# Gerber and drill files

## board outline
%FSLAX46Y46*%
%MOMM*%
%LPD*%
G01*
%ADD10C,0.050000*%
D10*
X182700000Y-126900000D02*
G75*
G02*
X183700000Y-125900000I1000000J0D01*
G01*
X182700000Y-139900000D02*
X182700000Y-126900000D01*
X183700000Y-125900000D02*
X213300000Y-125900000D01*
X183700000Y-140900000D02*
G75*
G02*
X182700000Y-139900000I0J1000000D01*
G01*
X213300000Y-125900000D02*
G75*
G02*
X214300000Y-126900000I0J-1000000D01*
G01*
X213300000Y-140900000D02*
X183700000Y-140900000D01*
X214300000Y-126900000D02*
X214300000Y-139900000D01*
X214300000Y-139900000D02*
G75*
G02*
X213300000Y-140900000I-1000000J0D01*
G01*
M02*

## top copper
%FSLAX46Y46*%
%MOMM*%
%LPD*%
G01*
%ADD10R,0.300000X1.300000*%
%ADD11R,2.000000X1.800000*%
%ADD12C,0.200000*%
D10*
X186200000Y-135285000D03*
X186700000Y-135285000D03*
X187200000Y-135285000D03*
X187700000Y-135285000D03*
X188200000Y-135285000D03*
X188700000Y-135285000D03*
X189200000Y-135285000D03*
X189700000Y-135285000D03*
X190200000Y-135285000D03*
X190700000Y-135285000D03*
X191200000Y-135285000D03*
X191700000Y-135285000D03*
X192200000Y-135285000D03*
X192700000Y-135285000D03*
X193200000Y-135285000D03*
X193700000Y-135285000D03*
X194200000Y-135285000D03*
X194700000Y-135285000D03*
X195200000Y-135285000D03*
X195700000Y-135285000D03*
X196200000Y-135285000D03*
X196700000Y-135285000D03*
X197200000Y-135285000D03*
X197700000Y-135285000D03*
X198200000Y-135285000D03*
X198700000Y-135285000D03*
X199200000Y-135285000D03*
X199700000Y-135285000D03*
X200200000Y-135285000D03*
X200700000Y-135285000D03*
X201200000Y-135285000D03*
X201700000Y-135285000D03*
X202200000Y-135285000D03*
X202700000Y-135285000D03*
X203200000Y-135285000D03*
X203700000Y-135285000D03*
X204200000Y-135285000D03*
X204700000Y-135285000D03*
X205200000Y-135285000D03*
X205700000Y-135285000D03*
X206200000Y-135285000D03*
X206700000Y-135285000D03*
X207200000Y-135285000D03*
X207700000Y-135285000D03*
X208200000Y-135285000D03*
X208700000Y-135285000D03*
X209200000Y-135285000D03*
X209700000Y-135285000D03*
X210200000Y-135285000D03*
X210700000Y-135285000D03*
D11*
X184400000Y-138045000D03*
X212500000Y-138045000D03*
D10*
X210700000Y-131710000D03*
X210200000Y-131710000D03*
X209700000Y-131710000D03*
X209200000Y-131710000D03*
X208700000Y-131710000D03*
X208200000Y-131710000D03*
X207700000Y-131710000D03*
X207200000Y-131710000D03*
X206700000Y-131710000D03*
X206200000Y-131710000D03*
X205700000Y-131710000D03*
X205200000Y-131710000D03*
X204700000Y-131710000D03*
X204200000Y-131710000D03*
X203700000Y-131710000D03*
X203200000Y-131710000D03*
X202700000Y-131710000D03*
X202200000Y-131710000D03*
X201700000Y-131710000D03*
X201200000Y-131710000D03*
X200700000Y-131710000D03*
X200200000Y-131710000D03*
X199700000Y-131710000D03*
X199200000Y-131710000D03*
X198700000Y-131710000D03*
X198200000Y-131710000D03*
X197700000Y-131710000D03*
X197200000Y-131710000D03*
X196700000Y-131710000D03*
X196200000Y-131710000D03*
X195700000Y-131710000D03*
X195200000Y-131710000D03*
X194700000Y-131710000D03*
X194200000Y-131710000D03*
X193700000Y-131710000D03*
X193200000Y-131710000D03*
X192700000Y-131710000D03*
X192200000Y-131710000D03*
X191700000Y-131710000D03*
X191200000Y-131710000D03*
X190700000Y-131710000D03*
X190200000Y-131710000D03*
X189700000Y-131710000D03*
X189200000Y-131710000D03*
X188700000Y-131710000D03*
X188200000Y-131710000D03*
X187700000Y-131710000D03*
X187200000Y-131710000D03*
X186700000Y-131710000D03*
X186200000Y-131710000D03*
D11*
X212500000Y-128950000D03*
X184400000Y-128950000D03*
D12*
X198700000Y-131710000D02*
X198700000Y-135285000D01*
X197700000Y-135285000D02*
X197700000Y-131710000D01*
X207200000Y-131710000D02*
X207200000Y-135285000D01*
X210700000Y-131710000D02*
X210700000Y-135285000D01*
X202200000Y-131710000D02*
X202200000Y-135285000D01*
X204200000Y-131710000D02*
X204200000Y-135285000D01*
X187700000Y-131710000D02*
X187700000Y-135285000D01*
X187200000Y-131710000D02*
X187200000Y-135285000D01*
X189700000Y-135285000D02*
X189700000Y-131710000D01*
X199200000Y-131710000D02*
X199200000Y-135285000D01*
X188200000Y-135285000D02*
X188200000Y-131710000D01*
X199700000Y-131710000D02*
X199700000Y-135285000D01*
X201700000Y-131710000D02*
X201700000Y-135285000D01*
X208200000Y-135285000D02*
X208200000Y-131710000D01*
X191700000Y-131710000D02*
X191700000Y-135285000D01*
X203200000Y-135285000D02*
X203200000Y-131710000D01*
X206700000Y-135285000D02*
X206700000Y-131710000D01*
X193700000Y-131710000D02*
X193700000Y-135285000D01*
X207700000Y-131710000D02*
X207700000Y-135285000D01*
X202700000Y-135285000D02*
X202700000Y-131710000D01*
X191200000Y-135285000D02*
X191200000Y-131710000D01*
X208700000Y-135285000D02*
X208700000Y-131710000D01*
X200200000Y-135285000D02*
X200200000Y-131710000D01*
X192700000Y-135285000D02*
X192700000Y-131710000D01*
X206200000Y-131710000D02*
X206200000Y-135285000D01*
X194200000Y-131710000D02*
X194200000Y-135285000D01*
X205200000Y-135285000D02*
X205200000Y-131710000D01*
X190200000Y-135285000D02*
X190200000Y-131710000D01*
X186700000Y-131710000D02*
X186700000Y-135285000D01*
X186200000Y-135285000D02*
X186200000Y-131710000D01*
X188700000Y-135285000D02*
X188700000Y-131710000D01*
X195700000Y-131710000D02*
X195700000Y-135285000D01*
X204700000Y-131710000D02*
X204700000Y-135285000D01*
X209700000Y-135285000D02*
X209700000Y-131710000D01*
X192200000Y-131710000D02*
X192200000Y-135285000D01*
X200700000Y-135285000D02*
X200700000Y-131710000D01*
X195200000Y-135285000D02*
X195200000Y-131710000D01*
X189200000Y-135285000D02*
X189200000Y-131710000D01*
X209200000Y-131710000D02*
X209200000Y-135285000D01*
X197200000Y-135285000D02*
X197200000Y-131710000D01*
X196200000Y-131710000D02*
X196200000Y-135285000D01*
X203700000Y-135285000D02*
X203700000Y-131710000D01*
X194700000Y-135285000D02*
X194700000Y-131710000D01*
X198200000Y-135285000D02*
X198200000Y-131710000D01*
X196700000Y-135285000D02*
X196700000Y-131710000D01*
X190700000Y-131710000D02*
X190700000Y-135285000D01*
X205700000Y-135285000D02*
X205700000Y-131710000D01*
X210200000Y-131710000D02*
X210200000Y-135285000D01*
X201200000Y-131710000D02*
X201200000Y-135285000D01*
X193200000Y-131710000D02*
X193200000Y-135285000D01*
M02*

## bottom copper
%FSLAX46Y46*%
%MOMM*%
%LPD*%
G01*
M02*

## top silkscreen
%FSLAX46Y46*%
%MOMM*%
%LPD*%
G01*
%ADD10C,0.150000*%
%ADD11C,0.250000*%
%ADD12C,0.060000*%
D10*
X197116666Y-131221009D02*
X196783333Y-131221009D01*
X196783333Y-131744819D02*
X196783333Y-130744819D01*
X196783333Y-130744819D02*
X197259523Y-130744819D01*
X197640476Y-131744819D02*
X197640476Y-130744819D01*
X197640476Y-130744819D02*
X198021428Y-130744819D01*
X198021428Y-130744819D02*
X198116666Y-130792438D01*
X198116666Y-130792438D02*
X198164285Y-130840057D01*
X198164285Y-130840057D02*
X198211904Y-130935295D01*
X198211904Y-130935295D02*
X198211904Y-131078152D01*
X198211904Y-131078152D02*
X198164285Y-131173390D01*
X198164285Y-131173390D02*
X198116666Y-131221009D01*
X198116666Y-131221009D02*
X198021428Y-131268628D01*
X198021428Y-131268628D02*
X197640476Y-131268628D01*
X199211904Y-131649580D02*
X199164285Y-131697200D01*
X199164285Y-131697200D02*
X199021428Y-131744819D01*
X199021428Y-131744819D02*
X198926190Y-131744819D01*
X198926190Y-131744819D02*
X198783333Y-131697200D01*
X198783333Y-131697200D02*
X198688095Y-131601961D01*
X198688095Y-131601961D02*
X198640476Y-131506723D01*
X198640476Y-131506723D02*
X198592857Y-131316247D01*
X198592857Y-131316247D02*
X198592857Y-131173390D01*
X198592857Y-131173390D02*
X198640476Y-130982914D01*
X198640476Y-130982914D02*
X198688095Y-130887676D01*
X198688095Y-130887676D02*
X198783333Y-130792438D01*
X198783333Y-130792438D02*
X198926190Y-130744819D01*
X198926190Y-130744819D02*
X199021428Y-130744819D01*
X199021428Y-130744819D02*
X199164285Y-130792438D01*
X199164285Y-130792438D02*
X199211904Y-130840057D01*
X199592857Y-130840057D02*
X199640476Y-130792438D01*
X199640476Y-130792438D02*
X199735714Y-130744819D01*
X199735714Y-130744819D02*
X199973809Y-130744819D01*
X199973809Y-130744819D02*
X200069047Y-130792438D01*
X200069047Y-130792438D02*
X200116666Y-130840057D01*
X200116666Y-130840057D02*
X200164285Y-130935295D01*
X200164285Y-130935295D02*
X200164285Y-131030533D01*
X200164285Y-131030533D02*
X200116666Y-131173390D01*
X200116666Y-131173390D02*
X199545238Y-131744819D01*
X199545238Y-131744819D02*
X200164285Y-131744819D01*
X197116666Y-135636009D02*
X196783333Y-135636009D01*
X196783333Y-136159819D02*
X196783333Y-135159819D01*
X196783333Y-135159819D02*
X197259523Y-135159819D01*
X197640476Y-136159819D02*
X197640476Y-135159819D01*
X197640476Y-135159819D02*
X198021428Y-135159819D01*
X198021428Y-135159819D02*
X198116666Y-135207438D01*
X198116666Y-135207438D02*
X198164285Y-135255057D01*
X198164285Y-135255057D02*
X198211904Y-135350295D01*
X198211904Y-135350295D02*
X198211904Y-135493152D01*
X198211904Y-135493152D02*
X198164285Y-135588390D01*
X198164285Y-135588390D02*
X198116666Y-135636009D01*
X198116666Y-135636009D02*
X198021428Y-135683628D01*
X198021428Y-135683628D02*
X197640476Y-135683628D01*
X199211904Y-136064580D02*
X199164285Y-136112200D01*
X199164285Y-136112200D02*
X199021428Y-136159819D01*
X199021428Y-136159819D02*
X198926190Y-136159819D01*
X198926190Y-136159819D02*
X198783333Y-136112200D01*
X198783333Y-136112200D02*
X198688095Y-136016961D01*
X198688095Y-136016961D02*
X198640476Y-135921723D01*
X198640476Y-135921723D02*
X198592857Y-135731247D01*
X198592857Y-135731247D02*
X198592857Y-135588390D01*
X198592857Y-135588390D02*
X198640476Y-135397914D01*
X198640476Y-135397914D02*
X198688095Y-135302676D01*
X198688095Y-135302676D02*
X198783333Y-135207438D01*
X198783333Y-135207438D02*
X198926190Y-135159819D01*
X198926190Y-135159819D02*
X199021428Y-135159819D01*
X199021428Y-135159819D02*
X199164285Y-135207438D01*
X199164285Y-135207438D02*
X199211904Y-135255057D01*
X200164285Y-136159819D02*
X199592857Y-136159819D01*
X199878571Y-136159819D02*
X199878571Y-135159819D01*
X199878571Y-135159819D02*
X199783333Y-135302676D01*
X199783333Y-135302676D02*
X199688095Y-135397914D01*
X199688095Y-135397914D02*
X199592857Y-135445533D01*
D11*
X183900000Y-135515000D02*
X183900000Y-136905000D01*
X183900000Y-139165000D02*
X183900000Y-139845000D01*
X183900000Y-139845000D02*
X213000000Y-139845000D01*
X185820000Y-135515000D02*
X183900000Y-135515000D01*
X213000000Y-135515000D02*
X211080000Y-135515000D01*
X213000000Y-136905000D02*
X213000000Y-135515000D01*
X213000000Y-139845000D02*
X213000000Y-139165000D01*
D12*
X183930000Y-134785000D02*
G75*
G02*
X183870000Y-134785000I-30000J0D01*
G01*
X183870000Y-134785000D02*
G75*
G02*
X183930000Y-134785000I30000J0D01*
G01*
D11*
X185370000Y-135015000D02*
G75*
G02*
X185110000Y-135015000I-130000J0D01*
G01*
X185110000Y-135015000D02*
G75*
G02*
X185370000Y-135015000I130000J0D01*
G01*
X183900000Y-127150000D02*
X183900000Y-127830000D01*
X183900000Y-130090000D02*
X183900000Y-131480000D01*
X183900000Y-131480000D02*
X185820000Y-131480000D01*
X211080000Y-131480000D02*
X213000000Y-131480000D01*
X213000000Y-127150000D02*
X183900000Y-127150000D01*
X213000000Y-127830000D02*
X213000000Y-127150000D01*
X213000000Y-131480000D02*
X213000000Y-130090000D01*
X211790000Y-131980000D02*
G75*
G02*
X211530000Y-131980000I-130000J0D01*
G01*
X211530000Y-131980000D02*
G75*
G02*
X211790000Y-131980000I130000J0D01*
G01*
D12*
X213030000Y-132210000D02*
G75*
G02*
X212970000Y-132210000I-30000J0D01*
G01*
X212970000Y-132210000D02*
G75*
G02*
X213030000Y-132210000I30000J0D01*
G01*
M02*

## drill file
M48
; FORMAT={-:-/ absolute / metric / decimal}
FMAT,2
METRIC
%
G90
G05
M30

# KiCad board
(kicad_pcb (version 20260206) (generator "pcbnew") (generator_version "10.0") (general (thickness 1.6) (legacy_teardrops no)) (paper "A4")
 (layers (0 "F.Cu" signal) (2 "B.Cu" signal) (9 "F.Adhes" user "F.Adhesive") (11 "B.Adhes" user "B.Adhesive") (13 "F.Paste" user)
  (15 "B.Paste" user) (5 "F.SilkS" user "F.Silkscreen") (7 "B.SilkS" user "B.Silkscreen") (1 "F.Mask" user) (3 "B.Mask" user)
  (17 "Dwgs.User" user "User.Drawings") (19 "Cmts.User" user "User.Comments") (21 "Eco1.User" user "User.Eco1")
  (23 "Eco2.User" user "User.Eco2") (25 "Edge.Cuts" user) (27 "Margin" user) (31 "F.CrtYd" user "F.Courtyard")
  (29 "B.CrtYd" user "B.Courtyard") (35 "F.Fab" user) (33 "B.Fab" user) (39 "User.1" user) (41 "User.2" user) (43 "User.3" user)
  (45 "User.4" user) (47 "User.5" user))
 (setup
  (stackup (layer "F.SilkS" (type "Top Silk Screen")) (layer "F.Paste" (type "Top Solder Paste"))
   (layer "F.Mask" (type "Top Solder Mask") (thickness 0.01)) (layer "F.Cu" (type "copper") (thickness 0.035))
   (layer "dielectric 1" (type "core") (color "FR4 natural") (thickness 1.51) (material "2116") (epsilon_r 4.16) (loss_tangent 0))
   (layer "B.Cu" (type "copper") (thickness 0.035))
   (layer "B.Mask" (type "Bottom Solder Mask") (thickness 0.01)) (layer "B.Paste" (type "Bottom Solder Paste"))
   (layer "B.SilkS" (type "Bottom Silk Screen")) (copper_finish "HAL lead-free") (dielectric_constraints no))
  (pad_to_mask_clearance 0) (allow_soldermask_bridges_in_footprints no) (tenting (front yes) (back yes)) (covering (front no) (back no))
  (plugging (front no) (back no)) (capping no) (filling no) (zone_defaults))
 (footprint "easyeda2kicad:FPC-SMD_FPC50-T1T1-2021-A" (layer "F.Cu") (at 198.45 136.665)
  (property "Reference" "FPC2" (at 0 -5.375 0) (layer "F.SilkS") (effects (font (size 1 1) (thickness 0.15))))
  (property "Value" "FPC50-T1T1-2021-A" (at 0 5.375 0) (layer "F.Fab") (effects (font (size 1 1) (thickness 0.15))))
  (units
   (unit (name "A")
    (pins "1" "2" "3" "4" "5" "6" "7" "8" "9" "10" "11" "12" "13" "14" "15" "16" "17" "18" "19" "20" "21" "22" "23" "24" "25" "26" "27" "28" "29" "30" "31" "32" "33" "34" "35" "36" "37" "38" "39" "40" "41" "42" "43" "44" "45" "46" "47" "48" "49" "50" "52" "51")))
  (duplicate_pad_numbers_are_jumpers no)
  (fp_line (start -14.55 -1.15) (end -14.55 0.24) (stroke (width 0.25) (type solid)) (layer "F.SilkS"))
  (fp_line (start -14.55 2.5) (end -14.55 3.18) (stroke (width 0.25) (type solid)) (layer "F.SilkS"))
  (fp_line (start -14.55 3.18) (end 14.55 3.18) (stroke (width 0.25) (type solid)) (layer "F.SilkS"))
  (fp_line (start -12.63 -1.15) (end -14.55 -1.15) (stroke (width 0.25) (type solid)) (layer "F.SilkS"))
  (fp_line (start 14.55 -1.15) (end 12.63 -1.15) (stroke (width 0.25) (type solid)) (layer "F.SilkS"))
  (fp_line (start 14.55 0.24) (end 14.55 -1.15) (stroke (width 0.25) (type solid)) (layer "F.SilkS"))
  (fp_line (start 14.55 3.18) (end 14.55 2.5) (stroke (width 0.25) (type solid)) (layer "F.SilkS"))
  (fp_circle (center -14.55 -1.88) (end -14.52 -1.88) (stroke (width 0.06) (type solid)) (fill no) (layer "F.SilkS"))
  (fp_circle (center -13.21 -1.65) (end -13.08 -1.65) (stroke (width 0.25) (type solid)) (fill no) (layer "F.SilkS"))
  (pad "1" smd rect (at -12.25 -1.38 180) (size 0.3 1.3) (layers "F.Cu" "F.Mask" "F.Paste") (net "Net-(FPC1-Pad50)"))
  (pad "2" smd rect (at -11.75 -1.38 180) (size 0.3 1.3) (layers "F.Cu" "F.Mask" "F.Paste") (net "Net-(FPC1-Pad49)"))
  (pad "3" smd rect (at -11.25 -1.38 180) (size 0.3 1.3) (layers "F.Cu" "F.Mask" "F.Paste") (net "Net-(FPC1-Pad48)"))
  (pad "4" smd rect (at -10.75 -1.38 180) (size 0.3 1.3) (layers "F.Cu" "F.Mask" "F.Paste") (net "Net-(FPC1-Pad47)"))
  (pad "5" smd rect (at -10.25 -1.38 180) (size 0.3 1.3) (layers "F.Cu" "F.Mask" "F.Paste") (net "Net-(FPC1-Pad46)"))
  (pad "6" smd rect (at -9.75 -1.38 180) (size 0.3 1.3) (layers "F.Cu" "F.Mask" "F.Paste") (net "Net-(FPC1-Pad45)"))
  (pad "7" smd rect (at -9.25 -1.38 180) (size 0.3 1.3) (layers "F.Cu" "F.Mask" "F.Paste") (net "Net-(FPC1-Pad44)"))
  (pad "8" smd rect (at -8.75 -1.38 180) (size 0.3 1.3) (layers "F.Cu" "F.Mask" "F.Paste") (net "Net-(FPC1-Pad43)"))
  (pad "9" smd rect (at -8.25 -1.38 180) (size 0.3 1.3) (layers "F.Cu" "F.Mask" "F.Paste") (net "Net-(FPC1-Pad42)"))
  (pad "10" smd rect (at -7.75 -1.38 180) (size 0.3 1.3) (layers "F.Cu" "F.Mask" "F.Paste") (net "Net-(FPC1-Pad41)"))
  (pad "11" smd rect (at -7.25 -1.38 180) (size 0.3 1.3) (layers "F.Cu" "F.Mask" "F.Paste") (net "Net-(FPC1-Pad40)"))
  (pad "12" smd rect (at -6.75 -1.38 180) (size 0.3 1.3) (layers "F.Cu" "F.Mask" "F.Paste") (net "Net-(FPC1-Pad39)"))
  (pad "13" smd rect (at -6.25 -1.38 180) (size 0.3 1.3) (layers "F.Cu" "F.Mask" "F.Paste") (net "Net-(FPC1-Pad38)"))
  (pad "14" smd rect (at -5.75 -1.38 180) (size 0.3 1.3) (layers "F.Cu" "F.Mask" "F.Paste") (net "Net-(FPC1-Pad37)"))
  (pad "15" smd rect (at -5.25 -1.38 180) (size 0.3 1.3) (layers "F.Cu" "F.Mask" "F.Paste") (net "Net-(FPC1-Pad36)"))
  (pad "16" smd rect (at -4.75 -1.38 180) (size 0.3 1.3) (layers "F.Cu" "F.Mask" "F.Paste") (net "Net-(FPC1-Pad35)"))
  (pad "17" smd rect (at -4.25 -1.38 180) (size 0.3 1.3) (layers "F.Cu" "F.Mask" "F.Paste") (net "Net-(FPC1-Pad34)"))
  (pad "18" smd rect (at -3.75 -1.38 180) (size 0.3 1.3) (layers "F.Cu" "F.Mask" "F.Paste") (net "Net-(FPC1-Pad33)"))
  (pad "19" smd rect (at -3.25 -1.38 180) (size 0.3 1.3) (layers "F.Cu" "F.Mask" "F.Paste") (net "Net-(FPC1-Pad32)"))
  (pad "20" smd rect (at -2.75 -1.38 180) (size 0.3 1.3) (layers "F.Cu" "F.Mask" "F.Paste") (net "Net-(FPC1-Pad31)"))
  (pad "21" smd rect (at -2.25 -1.38 180) (size 0.3 1.3) (layers "F.Cu" "F.Mask" "F.Paste") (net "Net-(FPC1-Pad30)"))
  (pad "22" smd rect (at -1.75 -1.38 180) (size 0.3 1.3) (layers "F.Cu" "F.Mask" "F.Paste") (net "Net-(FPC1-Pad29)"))
  (pad "23" smd rect (at -1.25 -1.38 180) (size 0.3 1.3) (layers "F.Cu" "F.Mask" "F.Paste") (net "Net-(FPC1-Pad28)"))
  (pad "24" smd rect (at -0.75 -1.38 180) (size 0.3 1.3) (layers "F.Cu" "F.Mask" "F.Paste") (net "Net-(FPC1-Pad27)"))
  (pad "25" smd rect (at -0.25 -1.38 180) (size 0.3 1.3) (layers "F.Cu" "F.Mask" "F.Paste") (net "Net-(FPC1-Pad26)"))
  (pad "26" smd rect (at 0.25 -1.38 180) (size 0.3 1.3) (layers "F.Cu" "F.Mask" "F.Paste") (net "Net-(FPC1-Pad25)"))
  (pad "27" smd rect (at 0.75 -1.38 180) (size 0.3 1.3) (layers "F.Cu" "F.Mask" "F.Paste") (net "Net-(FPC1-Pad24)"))
  (pad "28" smd rect (at 1.25 -1.38 180) (size 0.3 1.3) (layers "F.Cu" "F.Mask" "F.Paste") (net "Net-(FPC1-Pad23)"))
  (pad "29" smd rect (at 1.75 -1.38 180) (size 0.3 1.3) (layers "F.Cu" "F.Mask" "F.Paste") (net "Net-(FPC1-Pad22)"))
  (pad "30" smd rect (at 2.25 -1.38 180) (size 0.3 1.3) (layers "F.Cu" "F.Mask" "F.Paste") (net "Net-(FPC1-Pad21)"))
  (pad "31" smd rect (at 2.75 -1.38 180) (size 0.3 1.3) (layers "F.Cu" "F.Mask" "F.Paste") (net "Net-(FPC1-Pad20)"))
  (pad "32" smd rect (at 3.25 -1.38 180) (size 0.3 1.3) (layers "F.Cu" "F.Mask" "F.Paste") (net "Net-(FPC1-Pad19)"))
  (pad "33" smd rect (at 3.75 -1.38 180) (size 0.3 1.3) (layers "F.Cu" "F.Mask" "F.Paste") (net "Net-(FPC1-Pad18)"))
  (pad "34" smd rect (at 4.25 -1.38 180) (size 0.3 1.3) (layers "F.Cu" "F.Mask" "F.Paste") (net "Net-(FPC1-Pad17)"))
  (pad "35" smd rect (at 4.75 -1.38 180) (size 0.3 1.3) (layers "F.Cu" "F.Mask" "F.Paste") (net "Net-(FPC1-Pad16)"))
  (pad "36" smd rect (at 5.25 -1.38 180) (size 0.3 1.3) (layers "F.Cu" "F.Mask" "F.Paste") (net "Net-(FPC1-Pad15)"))
  (pad "37" smd rect (at 5.75 -1.38 180) (size 0.3 1.3) (layers "F.Cu" "F.Mask" "F.Paste") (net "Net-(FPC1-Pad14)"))
  (pad "38" smd rect (at 6.25 -1.38 180) (size 0.3 1.3) (layers "F.Cu" "F.Mask" "F.Paste") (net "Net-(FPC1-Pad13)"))
  (pad "39" smd rect (at 6.75 -1.38 180) (size 0.3 1.3) (layers "F.Cu" "F.Mask" "F.Paste") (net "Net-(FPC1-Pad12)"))
  (pad "40" smd rect (at 7.25 -1.38 180) (size 0.3 1.3) (layers "F.Cu" "F.Mask" "F.Paste") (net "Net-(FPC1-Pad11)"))
  (pad "41" smd rect (at 7.75 -1.38 180) (size 0.3 1.3) (layers "F.Cu" "F.Mask" "F.Paste") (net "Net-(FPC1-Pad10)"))
  (pad "42" smd rect (at 8.25 -1.38 180) (size 0.3 1.3) (layers "F.Cu" "F.Mask" "F.Paste") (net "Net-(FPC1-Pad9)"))
  (pad "43" smd rect (at 8.75 -1.38 180) (size 0.3 1.3) (layers "F.Cu" "F.Mask" "F.Paste") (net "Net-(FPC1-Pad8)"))
  (pad "44" smd rect (at 9.25 -1.38 180) (size 0.3 1.3) (layers "F.Cu" "F.Mask" "F.Paste") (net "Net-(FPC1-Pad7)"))
  (pad "45" smd rect (at 9.75 -1.38 180) (size 0.3 1.3) (layers "F.Cu" "F.Mask" "F.Paste") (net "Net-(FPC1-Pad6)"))
  (pad "46" smd rect (at 10.25 -1.38 180) (size 0.3 1.3) (layers "F.Cu" "F.Mask" "F.Paste") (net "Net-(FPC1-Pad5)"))
  (pad "47" smd rect (at 10.75 -1.38 180) (size 0.3 1.3) (layers "F.Cu" "F.Mask" "F.Paste") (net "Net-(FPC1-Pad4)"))
  (pad "48" smd rect (at 11.25 -1.38 180) (size 0.3 1.3) (layers "F.Cu" "F.Mask" "F.Paste") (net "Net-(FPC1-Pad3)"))
  (pad "49" smd rect (at 11.75 -1.38 180) (size 0.3 1.3) (layers "F.Cu" "F.Mask" "F.Paste") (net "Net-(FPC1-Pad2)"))
  (pad "50" smd rect (at 12.25 -1.38 180) (size 0.3 1.3) (layers "F.Cu" "F.Mask" "F.Paste") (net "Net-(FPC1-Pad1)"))
  (pad "51" smd rect (at -14.05 1.38 180) (size 2 1.8) (layers "F.Cu" "F.Mask" "F.Paste") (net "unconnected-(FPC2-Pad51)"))
  (pad "52" smd rect (at 14.05 1.38 180) (size 2 1.8) (layers "F.Cu" "F.Mask" "F.Paste") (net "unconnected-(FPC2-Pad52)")))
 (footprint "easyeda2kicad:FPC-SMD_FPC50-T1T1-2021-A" (layer "F.Cu") (at 198.45 130.33 180)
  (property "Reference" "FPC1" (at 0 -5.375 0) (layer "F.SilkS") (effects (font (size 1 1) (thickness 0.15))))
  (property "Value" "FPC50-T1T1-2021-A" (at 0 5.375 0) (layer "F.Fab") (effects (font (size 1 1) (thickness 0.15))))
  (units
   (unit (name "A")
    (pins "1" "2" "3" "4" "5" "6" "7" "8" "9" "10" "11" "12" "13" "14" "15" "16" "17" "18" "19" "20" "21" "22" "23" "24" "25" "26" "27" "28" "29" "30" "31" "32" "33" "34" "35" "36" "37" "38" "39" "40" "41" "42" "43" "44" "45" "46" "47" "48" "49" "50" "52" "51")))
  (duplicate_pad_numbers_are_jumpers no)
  (fp_line (start 14.55 3.18) (end 14.55 2.5) (stroke (width 0.25) (type solid)) (layer "F.SilkS"))
  (fp_line (start 14.55 0.24) (end 14.55 -1.15) (stroke (width 0.25) (type solid)) (layer "F.SilkS"))
  (fp_line (start 14.55 -1.15) (end 12.63 -1.15) (stroke (width 0.25) (type solid)) (layer "F.SilkS"))
  (fp_line (start -12.63 -1.15) (end -14.55 -1.15) (stroke (width 0.25) (type solid)) (layer "F.SilkS"))
  (fp_line (start -14.55 3.18) (end 14.55 3.18) (stroke (width 0.25) (type solid)) (layer "F.SilkS"))
  (fp_line (start -14.55 2.5) (end -14.55 3.18) (stroke (width 0.25) (type solid)) (layer "F.SilkS"))
  (fp_line (start -14.55 -1.15) (end -14.55 0.24) (stroke (width 0.25) (type solid)) (layer "F.SilkS"))
  (fp_circle (center -13.21 -1.65) (end -13.08 -1.65) (stroke (width 0.25) (type solid)) (fill no) (layer "F.SilkS"))
  (fp_circle (center -14.55 -1.88) (end -14.52 -1.88) (stroke (width 0.06) (type solid)) (fill no) (layer "F.SilkS"))
  (pad "1" smd rect (at -12.25 -1.38) (size 0.3 1.3) (layers "F.Cu" "F.Mask" "F.Paste") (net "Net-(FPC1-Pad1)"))
  (pad "2" smd rect (at -11.75 -1.38) (size 0.3 1.3) (layers "F.Cu" "F.Mask" "F.Paste") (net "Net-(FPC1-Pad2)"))
  (pad "3" smd rect (at -11.25 -1.38) (size 0.3 1.3) (layers "F.Cu" "F.Mask" "F.Paste") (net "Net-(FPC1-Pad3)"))
  (pad "4" smd rect (at -10.75 -1.38) (size 0.3 1.3) (layers "F.Cu" "F.Mask" "F.Paste") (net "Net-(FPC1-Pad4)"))
  (pad "5" smd rect (at -10.25 -1.38) (size 0.3 1.3) (layers "F.Cu" "F.Mask" "F.Paste") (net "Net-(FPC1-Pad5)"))
  (pad "6" smd rect (at -9.75 -1.38) (size 0.3 1.3) (layers "F.Cu" "F.Mask" "F.Paste") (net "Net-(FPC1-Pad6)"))
  (pad "7" smd rect (at -9.25 -1.38) (size 0.3 1.3) (layers "F.Cu" "F.Mask" "F.Paste") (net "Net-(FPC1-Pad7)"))
  (pad "8" smd rect (at -8.75 -1.38) (size 0.3 1.3) (layers "F.Cu" "F.Mask" "F.Paste") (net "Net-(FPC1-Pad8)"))
  (pad "9" smd rect (at -8.25 -1.38) (size 0.3 1.3) (layers "F.Cu" "F.Mask" "F.Paste") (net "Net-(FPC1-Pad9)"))
  (pad "10" smd rect (at -7.75 -1.38) (size 0.3 1.3) (layers "F.Cu" "F.Mask" "F.Paste") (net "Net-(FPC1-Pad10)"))
  (pad "11" smd rect (at -7.25 -1.38) (size 0.3 1.3) (layers "F.Cu" "F.Mask" "F.Paste") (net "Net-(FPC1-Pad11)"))
  (pad "12" smd rect (at -6.75 -1.38) (size 0.3 1.3) (layers "F.Cu" "F.Mask" "F.Paste") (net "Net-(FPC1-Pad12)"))
  (pad "13" smd rect (at -6.25 -1.38) (size 0.3 1.3) (layers "F.Cu" "F.Mask" "F.Paste") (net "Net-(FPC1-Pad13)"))
  (pad "14" smd rect (at -5.75 -1.38) (size 0.3 1.3) (layers "F.Cu" "F.Mask" "F.Paste") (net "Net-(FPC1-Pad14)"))
  (pad "15" smd rect (at -5.25 -1.38) (size 0.3 1.3) (layers "F.Cu" "F.Mask" "F.Paste") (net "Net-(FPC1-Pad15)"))
  (pad "16" smd rect (at -4.75 -1.38) (size 0.3 1.3) (layers "F.Cu" "F.Mask" "F.Paste") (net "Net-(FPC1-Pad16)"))
  (pad "17" smd rect (at -4.25 -1.38) (size 0.3 1.3) (layers "F.Cu" "F.Mask" "F.Paste") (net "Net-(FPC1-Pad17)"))
  (pad "18" smd rect (at -3.75 -1.38) (size 0.3 1.3) (layers "F.Cu" "F.Mask" "F.Paste") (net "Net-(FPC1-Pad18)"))
  (pad "19" smd rect (at -3.25 -1.38) (size 0.3 1.3) (layers "F.Cu" "F.Mask" "F.Paste") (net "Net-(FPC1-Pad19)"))
  (pad "20" smd rect (at -2.75 -1.38) (size 0.3 1.3) (layers "F.Cu" "F.Mask" "F.Paste") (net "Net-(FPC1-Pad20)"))
  (pad "21" smd rect (at -2.25 -1.38) (size 0.3 1.3) (layers "F.Cu" "F.Mask" "F.Paste") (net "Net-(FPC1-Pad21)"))
  (pad "22" smd rect (at -1.75 -1.38) (size 0.3 1.3) (layers "F.Cu" "F.Mask" "F.Paste") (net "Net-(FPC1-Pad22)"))
  (pad "23" smd rect (at -1.25 -1.38) (size 0.3 1.3) (layers "F.Cu" "F.Mask" "F.Paste") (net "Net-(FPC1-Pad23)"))
  (pad "24" smd rect (at -0.75 -1.38) (size 0.3 1.3) (layers "F.Cu" "F.Mask" "F.Paste") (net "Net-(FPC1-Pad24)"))
  (pad "25" smd rect (at -0.25 -1.38) (size 0.3 1.3) (layers "F.Cu" "F.Mask" "F.Paste") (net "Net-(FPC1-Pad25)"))
  (pad "26" smd rect (at 0.25 -1.38) (size 0.3 1.3) (layers "F.Cu" "F.Mask" "F.Paste") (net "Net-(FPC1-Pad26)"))
  (pad "27" smd rect (at 0.75 -1.38) (size 0.3 1.3) (layers "F.Cu" "F.Mask" "F.Paste") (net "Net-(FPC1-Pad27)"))
  (pad "28" smd rect (at 1.25 -1.38) (size 0.3 1.3) (layers "F.Cu" "F.Mask" "F.Paste") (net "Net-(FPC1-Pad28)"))
  (pad "29" smd rect (at 1.75 -1.38) (size 0.3 1.3) (layers "F.Cu" "F.Mask" "F.Paste") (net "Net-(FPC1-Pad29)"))
  (pad "30" smd rect (at 2.25 -1.38) (size 0.3 1.3) (layers "F.Cu" "F.Mask" "F.Paste") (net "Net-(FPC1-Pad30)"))
  (pad "31" smd rect (at 2.75 -1.38) (size 0.3 1.3) (layers "F.Cu" "F.Mask" "F.Paste") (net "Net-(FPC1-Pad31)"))
  (pad "32" smd rect (at 3.25 -1.38) (size 0.3 1.3) (layers "F.Cu" "F.Mask" "F.Paste") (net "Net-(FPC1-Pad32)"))
  (pad "33" smd rect (at 3.75 -1.38) (size 0.3 1.3) (layers "F.Cu" "F.Mask" "F.Paste") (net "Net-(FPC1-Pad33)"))
  (pad "34" smd rect (at 4.25 -1.38) (size 0.3 1.3) (layers "F.Cu" "F.Mask" "F.Paste") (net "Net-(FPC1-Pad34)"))
  (pad "35" smd rect (at 4.75 -1.38) (size 0.3 1.3) (layers "F.Cu" "F.Mask" "F.Paste") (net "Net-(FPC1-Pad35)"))
  (pad "36" smd rect (at 5.25 -1.38) (size 0.3 1.3) (layers "F.Cu" "F.Mask" "F.Paste") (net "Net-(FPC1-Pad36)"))
  (pad "37" smd rect (at 5.75 -1.38) (size 0.3 1.3) (layers "F.Cu" "F.Mask" "F.Paste") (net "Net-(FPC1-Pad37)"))
  (pad "38" smd rect (at 6.25 -1.38) (size 0.3 1.3) (layers "F.Cu" "F.Mask" "F.Paste") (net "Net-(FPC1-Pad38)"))
  (pad "39" smd rect (at 6.75 -1.38) (size 0.3 1.3) (layers "F.Cu" "F.Mask" "F.Paste") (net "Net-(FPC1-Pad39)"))
  (pad "40" smd rect (at 7.25 -1.38) (size 0.3 1.3) (layers "F.Cu" "F.Mask" "F.Paste") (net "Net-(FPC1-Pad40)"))
  (pad "41" smd rect (at 7.75 -1.38) (size 0.3 1.3) (layers "F.Cu" "F.Mask" "F.Paste") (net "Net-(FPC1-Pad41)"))
  (pad "42" smd rect (at 8.25 -1.38) (size 0.3 1.3) (layers "F.Cu" "F.Mask" "F.Paste") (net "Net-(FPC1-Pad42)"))
  (pad "43" smd rect (at 8.75 -1.38) (size 0.3 1.3) (layers "F.Cu" "F.Mask" "F.Paste") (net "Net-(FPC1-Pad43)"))
  (pad "44" smd rect (at 9.25 -1.38) (size 0.3 1.3) (layers "F.Cu" "F.Mask" "F.Paste") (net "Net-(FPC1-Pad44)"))
  (pad "45" smd rect (at 9.75 -1.38) (size 0.3 1.3) (layers "F.Cu" "F.Mask" "F.Paste") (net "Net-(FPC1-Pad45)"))
  (pad "46" smd rect (at 10.25 -1.38) (size 0.3 1.3) (layers "F.Cu" "F.Mask" "F.Paste") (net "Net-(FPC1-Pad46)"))
  (pad "47" smd rect (at 10.75 -1.38) (size 0.3 1.3) (layers "F.Cu" "F.Mask" "F.Paste") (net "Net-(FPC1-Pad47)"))
  (pad "48" smd rect (at 11.25 -1.38) (size 0.3 1.3) (layers "F.Cu" "F.Mask" "F.Paste") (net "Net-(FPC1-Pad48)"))
  (pad "49" smd rect (at 11.75 -1.38) (size 0.3 1.3) (layers "F.Cu" "F.Mask" "F.Paste") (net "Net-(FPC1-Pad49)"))
  (pad "50" smd rect (at 12.25 -1.38) (size 0.3 1.3) (layers "F.Cu" "F.Mask" "F.Paste") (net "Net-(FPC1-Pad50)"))
  (pad "51" smd rect (at -14.05 1.38) (size 2 1.8) (layers "F.Cu" "F.Mask" "F.Paste") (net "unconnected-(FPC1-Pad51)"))
  (pad "52" smd rect (at 14.05 1.38) (size 2 1.8) (layers "F.Cu" "F.Mask" "F.Paste") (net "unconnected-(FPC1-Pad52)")))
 (gr_arc (start 182.7 126.9) (mid 182.992893 126.192893) (end 183.7 125.9) (stroke (width 0.05) (type default)) (layer "Edge.Cuts"))
 (gr_line (start 182.7 139.9) (end 182.7 126.9) (stroke (width 0.05) (type default)) (layer "Edge.Cuts"))
 (gr_line (start 183.7 125.9) (end 213.3 125.9) (stroke (width 0.05) (type default)) (layer "Edge.Cuts"))
 (gr_arc (start 183.7 140.9) (mid 182.992893 140.607107) (end 182.7 139.9) (stroke (width 0.05) (type default)) (layer "Edge.Cuts"))
 (gr_arc (start 213.3 125.9) (mid 214.007107 126.192893) (end 214.3 126.9) (stroke (width 0.05) (type default)) (layer "Edge.Cuts"))
 (gr_line (start 213.3 140.9) (end 183.7 140.9) (stroke (width 0.05) (type default)) (layer "Edge.Cuts"))
 (gr_line (start 214.3 126.9) (end 214.3 139.9) (stroke (width 0.05) (type default)) (layer "Edge.Cuts"))
 (gr_arc (start 214.3 139.9) (mid 214.007107 140.607107) (end 213.3 140.9) (stroke (width 0.05) (type default)) (layer "Edge.Cuts"))
 (segment (start 198.7 131.71) (end 198.7 135.285) (width 0.2) (layer "F.Cu") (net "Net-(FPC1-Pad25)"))
 (segment (start 197.7 135.285) (end 197.7 131.71) (width 0.2) (layer "F.Cu") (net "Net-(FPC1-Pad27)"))
 (segment (start 207.2 131.71) (end 207.2 135.285) (width 0.2) (layer "F.Cu") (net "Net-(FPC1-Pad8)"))
 (segment (start 210.7 131.71) (end 210.7 135.285) (width 0.2) (layer "F.Cu") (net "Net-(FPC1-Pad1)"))
 (segment (start 202.2 131.71) (end 202.2 135.285) (width 0.2) (layer "F.Cu") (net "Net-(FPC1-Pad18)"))
 (segment (start 204.2 131.71) (end 204.2 135.285) (width 0.2) (layer "F.Cu") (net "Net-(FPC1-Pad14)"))
 (segment (start 187.7 131.71) (end 187.7 135.285) (width 0.2) (layer "F.Cu") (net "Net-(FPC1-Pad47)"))
 (segment (start 187.2 131.71) (end 187.2 135.285) (width 0.2) (layer "F.Cu") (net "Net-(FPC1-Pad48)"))
 (segment (start 189.7 135.285) (end 189.7 131.71) (width 0.2) (layer "F.Cu") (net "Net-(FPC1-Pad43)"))
 (segment (start 199.2 131.71) (end 199.2 135.285) (width 0.2) (layer "F.Cu") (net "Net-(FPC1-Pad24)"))
 (segment (start 188.2 135.285) (end 188.2 131.71) (width 0.2) (layer "F.Cu") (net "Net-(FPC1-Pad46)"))
 (segment (start 199.7 131.71) (end 199.7 135.285) (width 0.2) (layer "F.Cu") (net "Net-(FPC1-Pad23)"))
 (segment (start 201.7 131.71) (end 201.7 135.285) (width 0.2) (layer "F.Cu") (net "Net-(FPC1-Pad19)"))
 (segment (start 208.2 135.285) (end 208.2 131.71) (width 0.2) (layer "F.Cu") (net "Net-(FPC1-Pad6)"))
 (segment (start 191.7 131.71) (end 191.7 135.285) (width 0.2) (layer "F.Cu") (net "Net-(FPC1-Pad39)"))
 (segment (start 203.2 135.285) (end 203.2 131.71) (width 0.2) (layer "F.Cu") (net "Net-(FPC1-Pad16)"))
 (segment (start 206.7 135.285) (end 206.7 131.71) (width 0.2) (layer "F.Cu") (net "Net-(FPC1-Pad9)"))
 (segment (start 193.7 131.71) (end 193.7 135.285) (width 0.2) (layer "F.Cu") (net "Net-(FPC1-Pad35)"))
 (segment (start 207.7 131.71) (end 207.7 135.285) (width 0.2) (layer "F.Cu") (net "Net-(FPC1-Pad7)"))
 (segment (start 202.7 135.285) (end 202.7 131.71) (width 0.2) (layer "F.Cu") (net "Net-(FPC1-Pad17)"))
 (segment (start 191.2 135.285) (end 191.2 131.71) (width 0.2) (layer "F.Cu") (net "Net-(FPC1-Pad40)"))
 (segment (start 208.7 135.285) (end 208.7 131.71) (width 0.2) (layer "F.Cu") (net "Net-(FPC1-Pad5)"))
 (segment (start 200.2 135.285) (end 200.2 131.71) (width 0.2) (layer "F.Cu") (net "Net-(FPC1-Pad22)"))
 (segment (start 192.7 135.285) (end 192.7 131.71) (width 0.2) (layer "F.Cu") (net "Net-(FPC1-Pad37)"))
 (segment (start 206.2 131.71) (end 206.2 135.285) (width 0.2) (layer "F.Cu") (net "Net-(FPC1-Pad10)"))
 (segment (start 194.2 131.71) (end 194.2 135.285) (width 0.2) (layer "F.Cu") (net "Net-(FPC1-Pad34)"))
 (segment (start 205.2 135.285) (end 205.2 131.71) (width 0.2) (layer "F.Cu") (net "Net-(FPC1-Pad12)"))
 (segment (start 190.2 135.285) (end 190.2 131.71) (width 0.2) (layer "F.Cu") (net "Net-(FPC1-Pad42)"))
 (segment (start 186.7 131.71) (end 186.7 135.285) (width 0.2) (layer "F.Cu") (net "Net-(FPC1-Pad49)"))
 (segment (start 186.2 135.285) (end 186.2 131.71) (width 0.2) (layer "F.Cu") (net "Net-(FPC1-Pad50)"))
 (segment (start 188.7 135.285) (end 188.7 131.71) (width 0.2) (layer "F.Cu") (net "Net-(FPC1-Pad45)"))
 (segment (start 195.7 131.71) (end 195.7 135.285) (width 0.2) (layer "F.Cu") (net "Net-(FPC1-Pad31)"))
 (segment (start 204.7 131.71) (end 204.7 135.285) (width 0.2) (layer "F.Cu") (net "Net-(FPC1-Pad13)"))
 (segment (start 209.7 135.285) (end 209.7 131.71) (width 0.2) (layer "F.Cu") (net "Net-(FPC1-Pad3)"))
 (segment (start 192.2 131.71) (end 192.2 135.285) (width 0.2) (layer "F.Cu") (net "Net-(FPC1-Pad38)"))
 (segment (start 200.7 135.285) (end 200.7 131.71) (width 0.2) (layer "F.Cu") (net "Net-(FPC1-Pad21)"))
 (segment (start 195.2 135.285) (end 195.2 131.71) (width 0.2) (layer "F.Cu") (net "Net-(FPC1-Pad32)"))
 (segment (start 189.2 135.285) (end 189.2 131.71) (width 0.2) (layer "F.Cu") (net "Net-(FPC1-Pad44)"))
 (segment (start 209.2 131.71) (end 209.2 135.285) (width 0.2) (layer "F.Cu") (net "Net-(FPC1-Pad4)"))
 (segment (start 197.2 135.285) (end 197.2 131.71) (width 0.2) (layer "F.Cu") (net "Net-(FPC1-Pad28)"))
 (segment (start 196.2 131.71) (end 196.2 135.285) (width 0.2) (layer "F.Cu") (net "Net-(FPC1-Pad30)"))
 (segment (start 203.7 135.285) (end 203.7 131.71) (width 0.2) (layer "F.Cu") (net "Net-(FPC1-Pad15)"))
 (segment (start 194.7 135.285) (end 194.7 131.71) (width 0.2) (layer "F.Cu") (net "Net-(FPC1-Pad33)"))
 (segment (start 198.2 135.285) (end 198.2 131.71) (width 0.2) (layer "F.Cu") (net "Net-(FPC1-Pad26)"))
 (segment (start 196.7 135.285) (end 196.7 131.71) (width 0.2) (layer "F.Cu") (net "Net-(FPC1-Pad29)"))
 (segment (start 190.7 131.71) (end 190.7 135.285) (width 0.2) (layer "F.Cu") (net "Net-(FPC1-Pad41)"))
 (segment (start 205.7 135.285) (end 205.7 131.71) (width 0.2) (layer "F.Cu") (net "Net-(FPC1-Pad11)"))
 (segment (start 210.2 131.71) (end 210.2 135.285) (width 0.2) (layer "F.Cu") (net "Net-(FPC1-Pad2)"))
 (segment (start 201.2 131.71) (end 201.2 135.285) (width 0.2) (layer "F.Cu") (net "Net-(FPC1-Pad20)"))
 (segment (start 193.2 131.71) (end 193.2 135.285) (width 0.2) (layer "F.Cu") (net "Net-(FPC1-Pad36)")))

